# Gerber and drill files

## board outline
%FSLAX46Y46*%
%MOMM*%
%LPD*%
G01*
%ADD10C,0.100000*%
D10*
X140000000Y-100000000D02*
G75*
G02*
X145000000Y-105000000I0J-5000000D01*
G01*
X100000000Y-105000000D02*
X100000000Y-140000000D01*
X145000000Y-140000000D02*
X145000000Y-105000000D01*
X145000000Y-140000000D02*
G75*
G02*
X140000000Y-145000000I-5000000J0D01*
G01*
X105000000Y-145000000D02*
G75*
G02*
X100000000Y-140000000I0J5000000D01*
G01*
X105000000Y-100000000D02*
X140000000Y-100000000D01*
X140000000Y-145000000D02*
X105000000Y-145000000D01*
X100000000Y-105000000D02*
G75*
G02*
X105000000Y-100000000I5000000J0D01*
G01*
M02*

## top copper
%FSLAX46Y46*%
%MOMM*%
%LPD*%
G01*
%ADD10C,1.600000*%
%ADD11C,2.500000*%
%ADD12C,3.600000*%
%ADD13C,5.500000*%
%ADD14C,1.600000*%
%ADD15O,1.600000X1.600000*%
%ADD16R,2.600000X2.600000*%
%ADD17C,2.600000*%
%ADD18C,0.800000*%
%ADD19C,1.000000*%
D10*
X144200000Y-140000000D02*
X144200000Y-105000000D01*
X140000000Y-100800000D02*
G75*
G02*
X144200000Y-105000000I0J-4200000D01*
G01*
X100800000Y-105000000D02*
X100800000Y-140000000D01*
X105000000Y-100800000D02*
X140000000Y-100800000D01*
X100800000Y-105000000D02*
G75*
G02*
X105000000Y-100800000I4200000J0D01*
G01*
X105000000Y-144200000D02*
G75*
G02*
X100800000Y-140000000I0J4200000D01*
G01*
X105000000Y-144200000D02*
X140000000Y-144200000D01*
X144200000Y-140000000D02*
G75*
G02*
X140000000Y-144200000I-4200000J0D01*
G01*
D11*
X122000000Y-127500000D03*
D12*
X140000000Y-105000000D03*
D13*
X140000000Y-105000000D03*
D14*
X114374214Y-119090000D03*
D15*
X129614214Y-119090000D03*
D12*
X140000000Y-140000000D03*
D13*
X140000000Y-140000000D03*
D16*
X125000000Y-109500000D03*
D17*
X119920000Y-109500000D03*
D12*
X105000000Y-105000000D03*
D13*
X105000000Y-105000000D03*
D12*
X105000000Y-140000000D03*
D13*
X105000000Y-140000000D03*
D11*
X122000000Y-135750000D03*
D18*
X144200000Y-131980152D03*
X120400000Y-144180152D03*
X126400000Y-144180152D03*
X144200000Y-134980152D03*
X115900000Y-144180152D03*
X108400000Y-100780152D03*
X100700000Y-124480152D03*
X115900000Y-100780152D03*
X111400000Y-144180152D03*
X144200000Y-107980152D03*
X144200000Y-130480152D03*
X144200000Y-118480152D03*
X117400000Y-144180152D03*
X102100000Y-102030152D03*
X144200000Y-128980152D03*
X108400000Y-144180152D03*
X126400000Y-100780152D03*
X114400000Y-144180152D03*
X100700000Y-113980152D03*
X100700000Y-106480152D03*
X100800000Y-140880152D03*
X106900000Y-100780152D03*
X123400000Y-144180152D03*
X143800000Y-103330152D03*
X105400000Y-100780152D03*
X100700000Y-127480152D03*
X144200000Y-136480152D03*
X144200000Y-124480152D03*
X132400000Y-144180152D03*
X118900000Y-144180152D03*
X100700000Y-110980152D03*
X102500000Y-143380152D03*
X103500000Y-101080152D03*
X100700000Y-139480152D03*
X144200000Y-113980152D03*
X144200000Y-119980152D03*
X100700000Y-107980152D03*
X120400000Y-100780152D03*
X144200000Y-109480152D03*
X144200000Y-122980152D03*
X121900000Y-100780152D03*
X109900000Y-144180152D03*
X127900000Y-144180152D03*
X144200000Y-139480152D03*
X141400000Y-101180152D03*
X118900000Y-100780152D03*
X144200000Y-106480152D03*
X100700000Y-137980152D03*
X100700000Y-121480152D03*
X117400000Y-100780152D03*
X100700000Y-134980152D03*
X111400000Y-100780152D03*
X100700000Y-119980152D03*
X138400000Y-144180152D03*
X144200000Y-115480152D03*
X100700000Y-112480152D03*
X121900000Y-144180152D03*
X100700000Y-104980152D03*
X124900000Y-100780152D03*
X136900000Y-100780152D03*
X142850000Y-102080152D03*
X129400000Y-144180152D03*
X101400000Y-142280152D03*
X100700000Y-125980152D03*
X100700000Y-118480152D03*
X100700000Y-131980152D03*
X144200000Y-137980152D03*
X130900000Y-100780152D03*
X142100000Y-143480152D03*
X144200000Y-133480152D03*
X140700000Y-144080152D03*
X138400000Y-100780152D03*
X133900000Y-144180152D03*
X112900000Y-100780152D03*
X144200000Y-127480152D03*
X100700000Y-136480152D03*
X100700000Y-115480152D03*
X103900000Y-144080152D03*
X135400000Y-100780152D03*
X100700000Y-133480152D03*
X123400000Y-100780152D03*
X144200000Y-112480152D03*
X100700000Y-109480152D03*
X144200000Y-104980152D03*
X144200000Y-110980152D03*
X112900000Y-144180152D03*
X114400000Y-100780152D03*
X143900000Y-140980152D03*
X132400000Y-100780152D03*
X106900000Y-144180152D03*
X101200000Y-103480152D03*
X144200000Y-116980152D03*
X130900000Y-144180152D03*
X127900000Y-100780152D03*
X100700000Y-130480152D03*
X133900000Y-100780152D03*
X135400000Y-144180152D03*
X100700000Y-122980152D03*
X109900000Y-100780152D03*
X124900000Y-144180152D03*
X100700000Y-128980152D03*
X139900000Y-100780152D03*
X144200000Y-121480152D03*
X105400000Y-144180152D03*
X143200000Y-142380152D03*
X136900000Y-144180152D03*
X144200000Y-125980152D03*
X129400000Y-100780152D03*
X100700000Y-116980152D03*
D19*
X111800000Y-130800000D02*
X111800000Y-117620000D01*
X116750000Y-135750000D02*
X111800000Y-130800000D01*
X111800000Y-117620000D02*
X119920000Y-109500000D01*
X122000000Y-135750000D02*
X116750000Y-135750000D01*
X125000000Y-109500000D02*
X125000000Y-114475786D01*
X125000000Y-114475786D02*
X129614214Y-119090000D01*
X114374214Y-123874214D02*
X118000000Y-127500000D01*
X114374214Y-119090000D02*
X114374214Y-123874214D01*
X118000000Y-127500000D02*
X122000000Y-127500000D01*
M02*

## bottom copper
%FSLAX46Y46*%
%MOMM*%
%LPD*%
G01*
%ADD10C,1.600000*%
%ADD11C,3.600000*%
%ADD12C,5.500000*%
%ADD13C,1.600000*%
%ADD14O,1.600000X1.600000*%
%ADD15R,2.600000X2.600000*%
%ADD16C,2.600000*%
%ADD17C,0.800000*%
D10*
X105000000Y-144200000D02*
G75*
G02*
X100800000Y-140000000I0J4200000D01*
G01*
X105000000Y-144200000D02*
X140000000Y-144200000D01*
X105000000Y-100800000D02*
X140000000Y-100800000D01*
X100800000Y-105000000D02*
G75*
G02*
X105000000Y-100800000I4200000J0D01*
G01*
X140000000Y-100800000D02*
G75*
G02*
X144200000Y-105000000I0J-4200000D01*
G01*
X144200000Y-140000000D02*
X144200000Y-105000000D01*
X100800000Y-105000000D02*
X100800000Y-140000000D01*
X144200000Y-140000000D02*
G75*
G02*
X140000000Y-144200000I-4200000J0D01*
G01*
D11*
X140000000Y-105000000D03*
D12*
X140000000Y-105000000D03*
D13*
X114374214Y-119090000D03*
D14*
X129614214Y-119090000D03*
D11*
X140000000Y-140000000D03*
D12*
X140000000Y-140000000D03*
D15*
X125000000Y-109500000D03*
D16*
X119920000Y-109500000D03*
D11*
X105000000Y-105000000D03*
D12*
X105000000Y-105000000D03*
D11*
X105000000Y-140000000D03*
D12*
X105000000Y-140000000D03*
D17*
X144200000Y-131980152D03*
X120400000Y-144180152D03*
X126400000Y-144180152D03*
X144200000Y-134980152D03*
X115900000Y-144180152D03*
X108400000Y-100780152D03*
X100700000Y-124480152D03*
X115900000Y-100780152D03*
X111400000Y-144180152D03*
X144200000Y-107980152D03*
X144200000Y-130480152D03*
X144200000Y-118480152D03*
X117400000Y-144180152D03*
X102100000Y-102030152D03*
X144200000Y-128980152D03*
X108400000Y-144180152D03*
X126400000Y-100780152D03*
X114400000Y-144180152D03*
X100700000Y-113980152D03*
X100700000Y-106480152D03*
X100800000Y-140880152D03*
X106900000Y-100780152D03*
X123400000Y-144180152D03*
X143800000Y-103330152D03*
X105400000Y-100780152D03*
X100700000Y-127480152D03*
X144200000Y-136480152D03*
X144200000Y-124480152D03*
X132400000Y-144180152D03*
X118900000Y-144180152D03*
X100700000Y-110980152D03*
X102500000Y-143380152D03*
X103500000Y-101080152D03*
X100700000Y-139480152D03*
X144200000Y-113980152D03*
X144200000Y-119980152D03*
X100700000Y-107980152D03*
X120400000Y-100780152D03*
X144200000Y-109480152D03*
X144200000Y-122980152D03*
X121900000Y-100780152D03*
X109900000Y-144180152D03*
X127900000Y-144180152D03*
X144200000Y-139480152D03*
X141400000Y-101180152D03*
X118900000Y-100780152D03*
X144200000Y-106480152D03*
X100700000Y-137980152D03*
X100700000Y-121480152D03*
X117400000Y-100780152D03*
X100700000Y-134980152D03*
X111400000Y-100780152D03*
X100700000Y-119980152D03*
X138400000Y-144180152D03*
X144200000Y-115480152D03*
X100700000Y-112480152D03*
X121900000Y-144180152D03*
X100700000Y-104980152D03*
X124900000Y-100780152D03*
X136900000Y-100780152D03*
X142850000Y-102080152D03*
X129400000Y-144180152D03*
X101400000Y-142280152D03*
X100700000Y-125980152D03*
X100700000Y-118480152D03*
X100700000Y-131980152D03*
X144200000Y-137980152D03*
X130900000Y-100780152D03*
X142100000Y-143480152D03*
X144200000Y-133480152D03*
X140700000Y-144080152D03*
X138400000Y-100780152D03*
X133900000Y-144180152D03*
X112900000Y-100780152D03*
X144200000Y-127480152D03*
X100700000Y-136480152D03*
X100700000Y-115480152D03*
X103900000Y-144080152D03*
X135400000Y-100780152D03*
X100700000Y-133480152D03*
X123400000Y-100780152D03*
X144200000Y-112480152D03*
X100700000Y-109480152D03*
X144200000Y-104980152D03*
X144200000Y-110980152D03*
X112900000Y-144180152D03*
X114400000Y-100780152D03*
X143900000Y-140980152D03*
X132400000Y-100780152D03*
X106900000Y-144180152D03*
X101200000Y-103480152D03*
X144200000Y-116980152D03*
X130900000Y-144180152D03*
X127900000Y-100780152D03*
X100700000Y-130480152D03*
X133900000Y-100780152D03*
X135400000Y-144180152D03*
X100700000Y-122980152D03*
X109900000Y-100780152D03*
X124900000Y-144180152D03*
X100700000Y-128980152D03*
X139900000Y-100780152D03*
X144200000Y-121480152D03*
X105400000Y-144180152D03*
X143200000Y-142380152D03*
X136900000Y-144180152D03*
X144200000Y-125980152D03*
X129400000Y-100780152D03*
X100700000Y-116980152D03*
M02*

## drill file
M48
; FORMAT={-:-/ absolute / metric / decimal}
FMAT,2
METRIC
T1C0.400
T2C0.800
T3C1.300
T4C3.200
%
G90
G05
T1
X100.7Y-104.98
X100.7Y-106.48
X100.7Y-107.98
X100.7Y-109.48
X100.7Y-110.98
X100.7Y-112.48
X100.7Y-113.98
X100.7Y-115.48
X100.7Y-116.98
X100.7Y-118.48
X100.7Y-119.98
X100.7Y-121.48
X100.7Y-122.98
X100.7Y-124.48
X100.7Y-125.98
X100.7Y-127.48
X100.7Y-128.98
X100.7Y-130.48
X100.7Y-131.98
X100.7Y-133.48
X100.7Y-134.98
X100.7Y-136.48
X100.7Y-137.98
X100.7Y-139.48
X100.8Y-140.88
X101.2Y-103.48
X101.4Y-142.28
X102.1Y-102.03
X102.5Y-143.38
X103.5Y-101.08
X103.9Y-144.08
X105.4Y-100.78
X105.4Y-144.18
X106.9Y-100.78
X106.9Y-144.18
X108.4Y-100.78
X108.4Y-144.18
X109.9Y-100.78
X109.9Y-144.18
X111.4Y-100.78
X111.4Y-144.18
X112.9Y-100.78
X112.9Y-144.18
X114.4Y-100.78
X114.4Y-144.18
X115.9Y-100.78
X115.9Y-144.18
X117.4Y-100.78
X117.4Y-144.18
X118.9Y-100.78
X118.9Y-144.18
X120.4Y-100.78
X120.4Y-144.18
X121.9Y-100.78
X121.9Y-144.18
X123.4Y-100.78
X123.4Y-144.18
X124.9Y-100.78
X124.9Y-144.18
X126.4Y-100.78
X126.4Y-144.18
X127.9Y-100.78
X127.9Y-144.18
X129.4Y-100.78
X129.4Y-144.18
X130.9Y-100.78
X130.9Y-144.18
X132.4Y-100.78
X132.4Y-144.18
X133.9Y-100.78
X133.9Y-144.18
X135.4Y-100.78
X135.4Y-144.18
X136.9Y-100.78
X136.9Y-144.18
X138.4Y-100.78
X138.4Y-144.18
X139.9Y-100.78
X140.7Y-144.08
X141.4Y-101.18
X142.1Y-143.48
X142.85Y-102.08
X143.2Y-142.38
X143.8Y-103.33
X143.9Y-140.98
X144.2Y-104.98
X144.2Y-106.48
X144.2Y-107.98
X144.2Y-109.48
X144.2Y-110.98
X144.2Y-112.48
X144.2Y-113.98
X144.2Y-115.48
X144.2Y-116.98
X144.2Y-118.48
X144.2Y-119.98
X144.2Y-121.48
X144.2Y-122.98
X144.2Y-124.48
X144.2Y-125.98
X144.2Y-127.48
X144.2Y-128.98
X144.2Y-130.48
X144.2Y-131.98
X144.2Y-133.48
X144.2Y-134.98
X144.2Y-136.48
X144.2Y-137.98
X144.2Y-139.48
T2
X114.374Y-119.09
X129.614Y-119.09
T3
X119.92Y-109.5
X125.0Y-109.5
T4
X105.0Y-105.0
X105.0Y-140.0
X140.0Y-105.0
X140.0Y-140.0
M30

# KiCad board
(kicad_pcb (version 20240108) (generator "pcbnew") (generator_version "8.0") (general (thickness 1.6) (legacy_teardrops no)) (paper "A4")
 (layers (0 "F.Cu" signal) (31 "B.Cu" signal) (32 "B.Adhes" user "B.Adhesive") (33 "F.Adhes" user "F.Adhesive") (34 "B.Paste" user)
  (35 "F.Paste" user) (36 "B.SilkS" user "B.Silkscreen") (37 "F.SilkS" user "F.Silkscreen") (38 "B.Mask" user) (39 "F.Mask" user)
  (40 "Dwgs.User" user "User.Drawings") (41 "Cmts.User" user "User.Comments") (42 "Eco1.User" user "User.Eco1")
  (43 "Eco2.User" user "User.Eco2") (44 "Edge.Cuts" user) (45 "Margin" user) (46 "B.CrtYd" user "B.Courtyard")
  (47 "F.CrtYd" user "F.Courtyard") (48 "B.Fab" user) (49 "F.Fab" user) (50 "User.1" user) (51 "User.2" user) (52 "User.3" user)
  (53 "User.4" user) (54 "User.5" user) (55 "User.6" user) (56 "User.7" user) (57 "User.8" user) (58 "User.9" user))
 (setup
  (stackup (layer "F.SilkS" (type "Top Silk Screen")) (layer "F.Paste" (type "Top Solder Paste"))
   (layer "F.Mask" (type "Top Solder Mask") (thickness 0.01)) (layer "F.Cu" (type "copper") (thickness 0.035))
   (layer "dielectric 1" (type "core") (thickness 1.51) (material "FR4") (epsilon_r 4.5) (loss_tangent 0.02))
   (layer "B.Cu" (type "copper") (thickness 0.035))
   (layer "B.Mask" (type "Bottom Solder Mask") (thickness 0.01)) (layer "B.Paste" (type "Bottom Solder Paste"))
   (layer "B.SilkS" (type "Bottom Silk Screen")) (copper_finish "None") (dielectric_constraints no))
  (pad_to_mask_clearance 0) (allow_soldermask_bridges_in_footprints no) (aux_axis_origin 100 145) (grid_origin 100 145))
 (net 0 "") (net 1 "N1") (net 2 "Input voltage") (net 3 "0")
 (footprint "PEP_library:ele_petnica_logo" (layer "F.Cu") (at 136 126.6)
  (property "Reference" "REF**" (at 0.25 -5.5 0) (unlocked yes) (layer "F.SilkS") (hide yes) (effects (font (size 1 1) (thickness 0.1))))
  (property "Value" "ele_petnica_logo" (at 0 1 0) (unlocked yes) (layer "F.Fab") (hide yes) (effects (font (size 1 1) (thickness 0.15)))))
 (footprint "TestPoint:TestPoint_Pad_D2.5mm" (layer "F.Cu") (at 122 127.5)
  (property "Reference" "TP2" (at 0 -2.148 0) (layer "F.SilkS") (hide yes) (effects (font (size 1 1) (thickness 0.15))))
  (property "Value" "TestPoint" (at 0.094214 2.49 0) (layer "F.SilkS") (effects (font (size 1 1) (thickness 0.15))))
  (pad "1" smd circle (at 0 0) (size 2.5 2.5) (layers "F.Cu" "F.Mask") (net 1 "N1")))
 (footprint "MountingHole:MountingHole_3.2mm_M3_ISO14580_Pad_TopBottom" (layer "F.Cu") (at 140 105)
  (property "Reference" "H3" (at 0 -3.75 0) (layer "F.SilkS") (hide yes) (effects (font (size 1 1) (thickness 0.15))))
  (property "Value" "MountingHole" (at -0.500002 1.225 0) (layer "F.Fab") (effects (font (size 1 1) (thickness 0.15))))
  (pad "1" thru_hole circle (at 0 0) (size 3.6 3.6) (drill 3.2) (layers "*.Cu" "*.Mask") (remove_unused_layers no))
  (pad "1" connect circle (at 0 0) (size 5.5 5.5) (layers "F.Cu" "F.Mask"))
  (pad "1" connect circle (at 0 0) (size 5.5 5.5) (layers "B.Cu" "B.Mask")))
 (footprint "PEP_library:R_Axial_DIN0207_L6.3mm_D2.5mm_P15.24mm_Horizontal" (layer "F.Cu") (at 114.374214 119.09)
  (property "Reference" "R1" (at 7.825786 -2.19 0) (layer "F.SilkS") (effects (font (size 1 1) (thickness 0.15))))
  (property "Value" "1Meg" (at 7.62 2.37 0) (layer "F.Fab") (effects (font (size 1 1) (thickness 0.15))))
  (pad "1" thru_hole circle (at 0 0) (size 1.6 1.6) (drill 0.8) (layers "*.Cu" "*.Mask") (remove_unused_layers no) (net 1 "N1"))
  (pad "2" thru_hole oval (at 15.24 0) (size 1.6 1.6) (drill 0.8) (layers "*.Cu" "*.Mask") (remove_unused_layers no) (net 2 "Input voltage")))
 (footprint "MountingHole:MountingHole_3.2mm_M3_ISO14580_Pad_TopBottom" (layer "F.Cu") (at 140 140)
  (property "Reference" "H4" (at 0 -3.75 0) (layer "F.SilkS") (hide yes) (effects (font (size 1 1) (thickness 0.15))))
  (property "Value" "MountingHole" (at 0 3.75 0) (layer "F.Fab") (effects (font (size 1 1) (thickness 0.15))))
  (pad "1" thru_hole circle (at 0 0) (size 3.6 3.6) (drill 3.2) (layers "*.Cu" "*.Mask") (remove_unused_layers no))
  (pad "1" connect circle (at 0 0) (size 5.5 5.5) (layers "F.Cu" "F.Mask"))
  (pad "1" connect circle (at 0 0) (size 5.5 5.5) (layers "B.Cu" "B.Mask")))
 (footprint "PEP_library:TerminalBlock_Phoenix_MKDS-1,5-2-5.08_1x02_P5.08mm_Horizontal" (layer "F.Cu") (at 125 109.5 180)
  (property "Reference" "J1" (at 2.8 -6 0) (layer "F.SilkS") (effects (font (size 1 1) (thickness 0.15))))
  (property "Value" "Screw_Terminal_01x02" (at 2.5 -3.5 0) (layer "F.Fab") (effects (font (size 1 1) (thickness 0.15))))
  (pad "1" thru_hole rect (at 0 0 180) (size 2.6 2.6) (drill 1.3) (layers "*.Cu" "*.Mask") (remove_unused_layers no) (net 2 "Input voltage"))
  (pad "2" thru_hole circle (at 5.08 0 180) (size 2.6 2.6) (drill 1.3) (layers "*.Cu" "*.Mask") (remove_unused_layers no) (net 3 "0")))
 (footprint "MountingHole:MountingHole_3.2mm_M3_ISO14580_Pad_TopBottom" (layer "F.Cu") (at 105 105)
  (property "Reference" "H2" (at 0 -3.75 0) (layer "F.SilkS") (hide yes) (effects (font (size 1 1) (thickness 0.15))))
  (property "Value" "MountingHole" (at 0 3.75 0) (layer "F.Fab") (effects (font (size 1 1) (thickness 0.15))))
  (pad "1" thru_hole circle (at 0 0) (size 3.6 3.6) (drill 3.2) (layers "*.Cu" "*.Mask") (remove_unused_layers no))
  (pad "1" connect circle (at 0 0) (size 5.5 5.5) (layers "F.Cu" "F.Mask"))
  (pad "1" connect circle (at 0 0) (size 5.5 5.5) (layers "B.Cu" "B.Mask")))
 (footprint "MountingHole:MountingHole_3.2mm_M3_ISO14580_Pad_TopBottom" (layer "F.Cu") (at 105 140 -90)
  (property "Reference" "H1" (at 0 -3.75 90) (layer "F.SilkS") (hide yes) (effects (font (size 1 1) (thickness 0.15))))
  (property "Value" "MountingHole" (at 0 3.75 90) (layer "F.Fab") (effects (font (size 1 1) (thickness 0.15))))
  (pad "1" thru_hole circle (at 0 0 270) (size 3.6 3.6) (drill 3.2) (layers "*.Cu" "*.Mask") (remove_unused_layers no))
  (pad "1" connect circle (at 0 0 270) (size 5.5 5.5) (layers "F.Cu" "F.Mask"))
  (pad "1" connect circle (at 0 0 270) (size 5.5 5.5) (layers "B.Cu" "B.Mask")))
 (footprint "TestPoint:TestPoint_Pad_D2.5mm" (layer "F.Cu") (at 122 135.75)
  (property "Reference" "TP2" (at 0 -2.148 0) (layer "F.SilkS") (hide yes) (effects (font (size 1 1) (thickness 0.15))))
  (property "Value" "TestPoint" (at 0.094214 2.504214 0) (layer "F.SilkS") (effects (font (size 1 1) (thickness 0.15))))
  (pad "2" smd circle (at 0 0) (size 2.5 2.5) (layers "F.Cu" "F.Mask") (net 3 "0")))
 (gr_line (start 144.2 140) (end 144.2 105) (locked yes) (stroke (width 1.6) (type default)) (layer "F.Cu"))
 (gr_arc (start 140 100.8) (mid 142.969848 102.030152) (end 144.2 105) (locked yes) (stroke (width 1.6) (type default)) (layer "F.Cu"))
 (gr_line (start 100.8 105) (end 100.8 140) (locked yes) (stroke (width 1.6) (type default)) (layer "F.Cu"))
 (gr_line (start 105 100.8) (end 140 100.8) (locked yes) (stroke (width 1.6) (type default)) (layer "F.Cu"))
 (gr_arc (start 100.8 105) (mid 102.030152 102.030152) (end 105 100.8) (locked yes) (stroke (width 1.6) (type default)) (layer "F.Cu"))
 (gr_arc (start 105 144.2) (mid 102.030152 142.969848) (end 100.8 140) (locked yes) (stroke (width 1.6) (type default)) (layer "F.Cu"))
 (gr_line (start 105 144.2) (end 140 144.2) (locked yes) (stroke (width 1.6) (type default)) (layer "F.Cu"))
 (gr_arc (start 144.2 140) (mid 142.969848 142.969848) (end 140 144.2) (locked yes) (stroke (width 1.6) (type default)) (layer "F.Cu"))
 (gr_arc (start 105 144.2) (mid 102.030154 142.969848) (end 100.8 140) (locked yes) (stroke (width 1.6) (type default)) (layer "B.Cu"))
 (gr_line (start 105 144.2) (end 140 144.2) (locked yes) (stroke (width 1.6) (type default)) (layer "B.Cu"))
 (gr_line (start 105 100.8) (end 140 100.8) (locked yes) (stroke (width 1.6) (type default)) (layer "B.Cu"))
 (gr_arc (start 100.8 105) (mid 102.030152 102.030152) (end 105 100.8) (locked yes) (stroke (width 1.6) (type default)) (layer "B.Cu"))
 (gr_arc (start 140 100.8) (mid 142.96985 102.030151) (end 144.2 105) (locked yes) (stroke (width 1.6) (type default)) (layer "B.Cu"))
 (gr_line (start 144.2 140) (end 144.2 105) (locked yes) (stroke (width 1.6) (type default)) (layer "B.Cu"))
 (gr_line (start 100.8 105) (end 100.8 140) (locked yes) (stroke (width 1.6) (type default)) (layer "B.Cu"))
 (gr_arc (start 144.2 140) (mid 142.969849 142.969849) (end 140 144.2) (locked yes) (stroke (width 1.6) (type default)) (layer "B.Cu"))
 (gr_arc (start 140 100) (mid 143.535534 101.464466) (end 145 105) (locked yes) (stroke (width 0.1) (type default)) (layer "Edge.Cuts"))
 (gr_line (start 100 105) (end 100 140) (locked yes) (stroke (width 0.1) (type default)) (layer "Edge.Cuts"))
 (gr_line (start 145 140) (end 145 105) (locked yes) (stroke (width 0.1) (type default)) (layer "Edge.Cuts"))
 (gr_arc (start 145 140) (mid 143.535534 143.535534) (end 140 145) (locked yes) (stroke (width 0.1) (type default)) (layer "Edge.Cuts"))
 (gr_arc (start 105 145) (mid 101.464466 143.535534) (end 100 140) (locked yes) (stroke (width 0.1) (type default)) (layer "Edge.Cuts"))
 (gr_line (start 105 100) (end 140 100) (locked yes) (stroke (width 0.1) (type default)) (layer "Edge.Cuts"))
 (gr_line (start 140 145) (end 105 145) (locked yes) (stroke (width 0.1) (type default)) (layer "Edge.Cuts"))
 (gr_arc (start 100 105) (mid 101.464466 101.464466) (end 105 100) (locked yes) (stroke (width 0.1) (type default)) (layer "Edge.Cuts"))
 (via (at 144.2 131.980152) (size 0.8) (drill 0.4) (layers "F.Cu" "B.Cu") (locked yes) (free yes) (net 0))
 (via (at 120.4 144.180152) (size 0.8) (drill 0.4) (layers "F.Cu" "B.Cu") (locked yes) (free yes) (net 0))
 (via (at 126.4 144.180152) (size 0.8) (drill 0.4) (layers "F.Cu" "B.Cu") (locked yes) (free yes) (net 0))
 (via (at 144.2 134.980152) (size 0.8) (drill 0.4) (layers "F.Cu" "B.Cu") (locked yes) (free yes) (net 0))
 (via (at 115.9 144.180152) (size 0.8) (drill 0.4) (layers "F.Cu" "B.Cu") (locked yes) (free yes) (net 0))
 (via (at 108.4 100.780152) (size 0.8) (drill 0.4) (layers "F.Cu" "B.Cu") (locked yes) (free yes) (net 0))
 (via (at 100.7 124.480152) (size 0.8) (drill 0.4) (layers "F.Cu" "B.Cu") (locked yes) (free yes) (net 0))
 (via (at 115.9 100.780152) (size 0.8) (drill 0.4) (layers "F.Cu" "B.Cu") (locked yes) (free yes) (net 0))
 (via (at 111.4 144.180152) (size 0.8) (drill 0.4) (layers "F.Cu" "B.Cu") (locked yes) (free yes) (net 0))
 (via (at 144.2 107.980152) (size 0.8) (drill 0.4) (layers "F.Cu" "B.Cu") (locked yes) (free yes) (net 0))
 (via (at 144.2 130.480152) (size 0.8) (drill 0.4) (layers "F.Cu" "B.Cu") (locked yes) (free yes) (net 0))
 (via (at 144.2 118.480152) (size 0.8) (drill 0.4) (layers "F.Cu" "B.Cu") (locked yes) (free yes) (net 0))
 (via (at 117.4 144.180152) (size 0.8) (drill 0.4) (layers "F.Cu" "B.Cu") (locked yes) (free yes) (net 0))
 (via (at 102.1 102.030152) (size 0.8) (drill 0.4) (layers "F.Cu" "B.Cu") (locked yes) (free yes) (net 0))
 (via (at 144.2 128.980152) (size 0.8) (drill 0.4) (layers "F.Cu" "B.Cu") (locked yes) (free yes) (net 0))
 (via (at 108.4 144.180152) (size 0.8) (drill 0.4) (layers "F.Cu" "B.Cu") (locked yes) (free yes) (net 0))
 (via (at 126.4 100.780152) (size 0.8) (drill 0.4) (layers "F.Cu" "B.Cu") (locked yes) (free yes) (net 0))
 (via (at 114.4 144.180152) (size 0.8) (drill 0.4) (layers "F.Cu" "B.Cu") (locked yes) (free yes) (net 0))
 (via (at 100.7 113.980152) (size 0.8) (drill 0.4) (layers "F.Cu" "B.Cu") (locked yes) (free yes) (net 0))
 (via (at 100.7 106.480152) (size 0.8) (drill 0.4) (layers "F.Cu" "B.Cu") (locked yes) (free yes) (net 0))
 (via (at 100.8 140.880152) (size 0.8) (drill 0.4) (layers "F.Cu" "B.Cu") (locked yes) (free yes) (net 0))
 (via (at 106.9 100.780152) (size 0.8) (drill 0.4) (layers "F.Cu" "B.Cu") (locked yes) (free yes) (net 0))
 (via (at 123.4 144.180152) (size 0.8) (drill 0.4) (layers "F.Cu" "B.Cu") (locked yes) (free yes) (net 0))
 (via (at 143.8 103.330152) (size 0.8) (drill 0.4) (layers "F.Cu" "B.Cu") (locked yes) (free yes) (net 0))
 (via (at 105.4 100.780152) (size 0.8) (drill 0.4) (layers "F.Cu" "B.Cu") (locked yes) (free yes) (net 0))
 (via (at 100.7 127.480152) (size 0.8) (drill 0.4) (layers "F.Cu" "B.Cu") (locked yes) (free yes) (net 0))
 (via (at 144.2 136.480152) (size 0.8) (drill 0.4) (layers "F.Cu" "B.Cu") (locked yes) (free yes) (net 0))
 (via (at 144.2 124.480152) (size 0.8) (drill 0.4) (layers "F.Cu" "B.Cu") (locked yes) (free yes) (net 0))
 (via (at 132.4 144.180152) (size 0.8) (drill 0.4) (layers "F.Cu" "B.Cu") (locked yes) (free yes) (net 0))
 (via (at 118.9 144.180152) (size 0.8) (drill 0.4) (layers "F.Cu" "B.Cu") (locked yes) (free yes) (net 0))
 (via (at 100.7 110.980152) (size 0.8) (drill 0.4) (layers "F.Cu" "B.Cu") (locked yes) (free yes) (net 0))
 (via (at 102.5 143.380152) (size 0.8) (drill 0.4) (layers "F.Cu" "B.Cu") (locked yes) (free yes) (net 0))
 (via (at 103.5 101.080152) (size 0.8) (drill 0.4) (layers "F.Cu" "B.Cu") (locked yes) (free yes) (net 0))
 (via (at 100.7 139.480152) (size 0.8) (drill 0.4) (layers "F.Cu" "B.Cu") (locked yes) (free yes) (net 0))
 (via (at 144.2 113.980152) (size 0.8) (drill 0.4) (layers "F.Cu" "B.Cu") (locked yes) (free yes) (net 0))
 (via (at 144.2 119.980152) (size 0.8) (drill 0.4) (layers "F.Cu" "B.Cu") (locked yes) (free yes) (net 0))
 (via (at 100.7 107.980152) (size 0.8) (drill 0.4) (layers "F.Cu" "B.Cu") (locked yes) (free yes) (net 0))
 (via (at 120.4 100.780152) (size 0.8) (drill 0.4) (layers "F.Cu" "B.Cu") (locked yes) (free yes) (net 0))
 (via (at 144.2 109.480152) (size 0.8) (drill 0.4) (layers "F.Cu" "B.Cu") (locked yes) (free yes) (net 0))
 (via (at 144.2 122.980152) (size 0.8) (drill 0.4) (layers "F.Cu" "B.Cu") (locked yes) (free yes) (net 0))
 (via (at 121.9 100.780152) (size 0.8) (drill 0.4) (layers "F.Cu" "B.Cu") (locked yes) (free yes) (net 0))
 (via (at 109.9 144.180152) (size 0.8) (drill 0.4) (layers "F.Cu" "B.Cu") (locked yes) (free yes) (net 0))
 (via (at 127.9 144.180152) (size 0.8) (drill 0.4) (layers "F.Cu" "B.Cu") (locked yes) (free yes) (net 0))
 (via (at 144.2 139.480152) (size 0.8) (drill 0.4) (layers "F.Cu" "B.Cu") (locked yes) (free yes) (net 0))
 (via (at 141.4 101.180152) (size 0.8) (drill 0.4) (layers "F.Cu" "B.Cu") (locked yes) (free yes) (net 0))
 (via (at 118.9 100.780152) (size 0.8) (drill 0.4) (layers "F.Cu" "B.Cu") (locked yes) (free yes) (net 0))
 (via (at 144.2 106.480152) (size 0.8) (drill 0.4) (layers "F.Cu" "B.Cu") (locked yes) (free yes) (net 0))
 (via (at 100.7 137.980152) (size 0.8) (drill 0.4) (layers "F.Cu" "B.Cu") (locked yes) (free yes) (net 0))
 (via (at 100.7 121.480152) (size 0.8) (drill 0.4) (layers "F.Cu" "B.Cu") (locked yes) (free yes) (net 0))
 (via (at 117.4 100.780152) (size 0.8) (drill 0.4) (layers "F.Cu" "B.Cu") (locked yes) (free yes) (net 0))
 (via (at 100.7 134.980152) (size 0.8) (drill 0.4) (layers "F.Cu" "B.Cu") (locked yes) (free yes) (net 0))
 (via (at 111.4 100.780152) (size 0.8) (drill 0.4) (layers "F.Cu" "B.Cu") (locked yes) (free yes) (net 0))
 (via (at 100.7 119.980152) (size 0.8) (drill 0.4) (layers "F.Cu" "B.Cu") (locked yes) (free yes) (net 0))
 (via (at 138.4 144.180152) (size 0.8) (drill 0.4) (layers "F.Cu" "B.Cu") (locked yes) (free yes) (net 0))
 (via (at 144.2 115.480152) (size 0.8) (drill 0.4) (layers "F.Cu" "B.Cu") (locked yes) (free yes) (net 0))
 (via (at 100.7 112.480152) (size 0.8) (drill 0.4) (layers "F.Cu" "B.Cu") (locked yes) (free yes) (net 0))
 (via (at 121.9 144.180152) (size 0.8) (drill 0.4) (layers "F.Cu" "B.Cu") (locked yes) (free yes) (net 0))
 (via (at 100.7 104.980152) (size 0.8) (drill 0.4) (layers "F.Cu" "B.Cu") (locked yes) (free yes) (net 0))
 (via (at 124.9 100.780152) (size 0.8) (drill 0.4) (layers "F.Cu" "B.Cu") (locked yes) (free yes) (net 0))
 (via (at 136.9 100.780152) (size 0.8) (drill 0.4) (layers "F.Cu" "B.Cu") (locked yes) (free yes) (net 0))
 (via (at 142.85 102.080152) (size 0.8) (drill 0.4) (layers "F.Cu" "B.Cu") (locked yes) (free yes) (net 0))
 (via (at 129.4 144.180152) (size 0.8) (drill 0.4) (layers "F.Cu" "B.Cu") (locked yes) (free yes) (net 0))
 (via (at 101.4 142.280152) (size 0.8) (drill 0.4) (layers "F.Cu" "B.Cu") (locked yes) (free yes) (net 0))
 (via (at 100.7 125.980152) (size 0.8) (drill 0.4) (layers "F.Cu" "B.Cu") (locked yes) (free yes) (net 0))
 (via (at 100.7 118.480152) (size 0.8) (drill 0.4) (layers "F.Cu" "B.Cu") (locked yes) (free yes) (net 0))
 (via (at 100.7 131.980152) (size 0.8) (drill 0.4) (layers "F.Cu" "B.Cu") (locked yes) (free yes) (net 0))
 (via (at 144.2 137.980152) (size 0.8) (drill 0.4) (layers "F.Cu" "B.Cu") (locked yes) (free yes) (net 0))
 (via (at 130.9 100.780152) (size 0.8) (drill 0.4) (layers "F.Cu" "B.Cu") (locked yes) (free yes) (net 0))
 (via (at 142.1 143.480152) (size 0.8) (drill 0.4) (layers "F.Cu" "B.Cu") (locked yes) (free yes) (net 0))
 (via (at 144.2 133.480152) (size 0.8) (drill 0.4) (layers "F.Cu" "B.Cu") (locked yes) (free yes) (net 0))
 (via (at 140.7 144.080152) (size 0.8) (drill 0.4) (layers "F.Cu" "B.Cu") (locked yes) (free yes) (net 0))
 (via (at 138.4 100.780152) (size 0.8) (drill 0.4) (layers "F.Cu" "B.Cu") (locked yes) (free yes) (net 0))
 (via (at 133.9 144.180152) (size 0.8) (drill 0.4) (layers "F.Cu" "B.Cu") (locked yes) (free yes) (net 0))
 (via (at 112.9 100.780152) (size 0.8) (drill 0.4) (layers "F.Cu" "B.Cu") (locked yes) (free yes) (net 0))
 (via (at 144.2 127.480152) (size 0.8) (drill 0.4) (layers "F.Cu" "B.Cu") (locked yes) (free yes) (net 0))
 (via (at 100.7 136.480152) (size 0.8) (drill 0.4) (layers "F.Cu" "B.Cu") (locked yes) (free yes) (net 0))
 (via (at 100.7 115.480152) (size 0.8) (drill 0.4) (layers "F.Cu" "B.Cu") (locked yes) (free yes) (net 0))
 (via (at 103.9 144.080152) (size 0.8) (drill 0.4) (layers "F.Cu" "B.Cu") (locked yes) (free yes) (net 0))
 (via (at 135.4 100.780152) (size 0.8) (drill 0.4) (layers "F.Cu" "B.Cu") (locked yes) (free yes) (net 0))
 (via (at 100.7 133.480152) (size 0.8) (drill 0.4) (layers "F.Cu" "B.Cu") (locked yes) (free yes) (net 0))
 (via (at 123.4 100.780152) (size 0.8) (drill 0.4) (layers "F.Cu" "B.Cu") (locked yes) (free yes) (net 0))
 (via (at 144.2 112.480152) (size 0.8) (drill 0.4) (layers "F.Cu" "B.Cu") (locked yes) (free yes) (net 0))
 (via (at 100.7 109.480152) (size 0.8) (drill 0.4) (layers "F.Cu" "B.Cu") (locked yes) (free yes) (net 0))
 (via (at 144.2 104.980152) (size 0.8) (drill 0.4) (layers "F.Cu" "B.Cu") (locked yes) (free yes) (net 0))
 (via (at 144.2 110.980152) (size 0.8) (drill 0.4) (layers "F.Cu" "B.Cu") (locked yes) (free yes) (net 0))
 (via (at 112.9 144.180152) (size 0.8) (drill 0.4) (layers "F.Cu" "B.Cu") (locked yes) (free yes) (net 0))
 (via (at 114.4 100.780152) (size 0.8) (drill 0.4) (layers "F.Cu" "B.Cu") (locked yes) (free yes) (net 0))
 (via (at 143.9 140.980152) (size 0.8) (drill 0.4) (layers "F.Cu" "B.Cu") (locked yes) (free yes) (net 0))
 (via (at 132.4 100.780152) (size 0.8) (drill 0.4) (layers "F.Cu" "B.Cu") (locked yes) (free yes) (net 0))
 (via (at 106.9 144.180152) (size 0.8) (drill 0.4) (layers "F.Cu" "B.Cu") (locked yes) (free yes) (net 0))
 (via (at 101.2 103.480152) (size 0.8) (drill 0.4) (layers "F.Cu" "B.Cu") (locked yes) (free yes) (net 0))
 (via (at 144.2 116.980152) (size 0.8) (drill 0.4) (layers "F.Cu" "B.Cu") (locked yes) (free yes) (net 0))
 (via (at 130.9 144.180152) (size 0.8) (drill 0.4) (layers "F.Cu" "B.Cu") (locked yes) (free yes) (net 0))
 (via (at 127.9 100.780152) (size 0.8) (drill 0.4) (layers "F.Cu" "B.Cu") (locked yes) (free yes) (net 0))
 (via (at 100.7 130.480152) (size 0.8) (drill 0.4) (layers "F.Cu" "B.Cu") (locked yes) (free yes) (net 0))
 (via (at 133.9 100.780152) (size 0.8) (drill 0.4) (layers "F.Cu" "B.Cu") (locked yes) (free yes) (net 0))
 (via (at 135.4 144.180152) (size 0.8) (drill 0.4) (layers "F.Cu" "B.Cu") (locked yes) (free yes) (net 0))
 (via (at 100.7 122.980152) (size 0.8) (drill 0.4) (layers "F.Cu" "B.Cu") (locked yes) (free yes) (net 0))
 (via (at 109.9 100.780152) (size 0.8) (drill 0.4) (layers "F.Cu" "B.Cu") (locked yes) (free yes) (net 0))
 (via (at 124.9 144.180152) (size 0.8) (drill 0.4) (layers "F.Cu" "B.Cu") (locked yes) (free yes) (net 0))
 (via (at 100.7 128.980152) (size 0.8) (drill 0.4) (layers "F.Cu" "B.Cu") (locked yes) (free yes) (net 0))
 (via (at 139.9 100.780152) (size 0.8) (drill 0.4) (layers "F.Cu" "B.Cu") (locked yes) (free yes) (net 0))
 (via (at 144.2 121.480152) (size 0.8) (drill 0.4) (layers "F.Cu" "B.Cu") (locked yes) (free yes) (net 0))
 (via (at 105.4 144.180152) (size 0.8) (drill 0.4) (layers "F.Cu" "B.Cu") (locked yes) (free yes) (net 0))
 (via (at 143.2 142.380152) (size 0.8) (drill 0.4) (layers "F.Cu" "B.Cu") (locked yes) (free yes) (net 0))
 (via (at 136.9 144.180152) (size 0.8) (drill 0.4) (layers "F.Cu" "B.Cu") (locked yes) (free yes) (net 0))
 (via (at 144.2 125.980152) (size 0.8) (drill 0.4) (layers "F.Cu" "B.Cu") (locked yes) (free yes) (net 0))
 (via (at 129.4 100.780152) (size 0.8) (drill 0.4) (layers "F.Cu" "B.Cu") (locked yes) (free yes) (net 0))
 (via (at 100.7 116.980152) (size 0.8) (drill 0.4) (layers "F.Cu" "B.Cu") (locked yes) (free yes) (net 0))
 (segment (start 111.8 130.8) (end 111.8 117.62) (width 1) (layer "F.Cu") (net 3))
 (segment (start 116.75 135.75) (end 111.8 130.8) (width 1) (layer "F.Cu") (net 3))
 (segment (start 111.8 117.62) (end 119.92 109.5) (width 1) (layer "F.Cu") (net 3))
 (segment (start 122 135.75) (end 116.75 135.75) (width 1) (layer "F.Cu") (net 3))
 (segment (start 125 109.5) (end 125 114.475786) (width 1) (layer "F.Cu") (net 2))
 (segment (start 125 114.475786) (end 129.614214 119.09) (width 1) (layer "F.Cu") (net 2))
 (segment (start 114.374214 123.874214) (end 118 127.5) (width 1) (layer "F.Cu") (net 1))
 (segment (start 114.374214 119.09) (end 114.374214 123.874214) (width 1) (layer "F.Cu") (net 1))
 (segment (start 118 127.5) (end 122 127.5) (width 1) (layer "F.Cu") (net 1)))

